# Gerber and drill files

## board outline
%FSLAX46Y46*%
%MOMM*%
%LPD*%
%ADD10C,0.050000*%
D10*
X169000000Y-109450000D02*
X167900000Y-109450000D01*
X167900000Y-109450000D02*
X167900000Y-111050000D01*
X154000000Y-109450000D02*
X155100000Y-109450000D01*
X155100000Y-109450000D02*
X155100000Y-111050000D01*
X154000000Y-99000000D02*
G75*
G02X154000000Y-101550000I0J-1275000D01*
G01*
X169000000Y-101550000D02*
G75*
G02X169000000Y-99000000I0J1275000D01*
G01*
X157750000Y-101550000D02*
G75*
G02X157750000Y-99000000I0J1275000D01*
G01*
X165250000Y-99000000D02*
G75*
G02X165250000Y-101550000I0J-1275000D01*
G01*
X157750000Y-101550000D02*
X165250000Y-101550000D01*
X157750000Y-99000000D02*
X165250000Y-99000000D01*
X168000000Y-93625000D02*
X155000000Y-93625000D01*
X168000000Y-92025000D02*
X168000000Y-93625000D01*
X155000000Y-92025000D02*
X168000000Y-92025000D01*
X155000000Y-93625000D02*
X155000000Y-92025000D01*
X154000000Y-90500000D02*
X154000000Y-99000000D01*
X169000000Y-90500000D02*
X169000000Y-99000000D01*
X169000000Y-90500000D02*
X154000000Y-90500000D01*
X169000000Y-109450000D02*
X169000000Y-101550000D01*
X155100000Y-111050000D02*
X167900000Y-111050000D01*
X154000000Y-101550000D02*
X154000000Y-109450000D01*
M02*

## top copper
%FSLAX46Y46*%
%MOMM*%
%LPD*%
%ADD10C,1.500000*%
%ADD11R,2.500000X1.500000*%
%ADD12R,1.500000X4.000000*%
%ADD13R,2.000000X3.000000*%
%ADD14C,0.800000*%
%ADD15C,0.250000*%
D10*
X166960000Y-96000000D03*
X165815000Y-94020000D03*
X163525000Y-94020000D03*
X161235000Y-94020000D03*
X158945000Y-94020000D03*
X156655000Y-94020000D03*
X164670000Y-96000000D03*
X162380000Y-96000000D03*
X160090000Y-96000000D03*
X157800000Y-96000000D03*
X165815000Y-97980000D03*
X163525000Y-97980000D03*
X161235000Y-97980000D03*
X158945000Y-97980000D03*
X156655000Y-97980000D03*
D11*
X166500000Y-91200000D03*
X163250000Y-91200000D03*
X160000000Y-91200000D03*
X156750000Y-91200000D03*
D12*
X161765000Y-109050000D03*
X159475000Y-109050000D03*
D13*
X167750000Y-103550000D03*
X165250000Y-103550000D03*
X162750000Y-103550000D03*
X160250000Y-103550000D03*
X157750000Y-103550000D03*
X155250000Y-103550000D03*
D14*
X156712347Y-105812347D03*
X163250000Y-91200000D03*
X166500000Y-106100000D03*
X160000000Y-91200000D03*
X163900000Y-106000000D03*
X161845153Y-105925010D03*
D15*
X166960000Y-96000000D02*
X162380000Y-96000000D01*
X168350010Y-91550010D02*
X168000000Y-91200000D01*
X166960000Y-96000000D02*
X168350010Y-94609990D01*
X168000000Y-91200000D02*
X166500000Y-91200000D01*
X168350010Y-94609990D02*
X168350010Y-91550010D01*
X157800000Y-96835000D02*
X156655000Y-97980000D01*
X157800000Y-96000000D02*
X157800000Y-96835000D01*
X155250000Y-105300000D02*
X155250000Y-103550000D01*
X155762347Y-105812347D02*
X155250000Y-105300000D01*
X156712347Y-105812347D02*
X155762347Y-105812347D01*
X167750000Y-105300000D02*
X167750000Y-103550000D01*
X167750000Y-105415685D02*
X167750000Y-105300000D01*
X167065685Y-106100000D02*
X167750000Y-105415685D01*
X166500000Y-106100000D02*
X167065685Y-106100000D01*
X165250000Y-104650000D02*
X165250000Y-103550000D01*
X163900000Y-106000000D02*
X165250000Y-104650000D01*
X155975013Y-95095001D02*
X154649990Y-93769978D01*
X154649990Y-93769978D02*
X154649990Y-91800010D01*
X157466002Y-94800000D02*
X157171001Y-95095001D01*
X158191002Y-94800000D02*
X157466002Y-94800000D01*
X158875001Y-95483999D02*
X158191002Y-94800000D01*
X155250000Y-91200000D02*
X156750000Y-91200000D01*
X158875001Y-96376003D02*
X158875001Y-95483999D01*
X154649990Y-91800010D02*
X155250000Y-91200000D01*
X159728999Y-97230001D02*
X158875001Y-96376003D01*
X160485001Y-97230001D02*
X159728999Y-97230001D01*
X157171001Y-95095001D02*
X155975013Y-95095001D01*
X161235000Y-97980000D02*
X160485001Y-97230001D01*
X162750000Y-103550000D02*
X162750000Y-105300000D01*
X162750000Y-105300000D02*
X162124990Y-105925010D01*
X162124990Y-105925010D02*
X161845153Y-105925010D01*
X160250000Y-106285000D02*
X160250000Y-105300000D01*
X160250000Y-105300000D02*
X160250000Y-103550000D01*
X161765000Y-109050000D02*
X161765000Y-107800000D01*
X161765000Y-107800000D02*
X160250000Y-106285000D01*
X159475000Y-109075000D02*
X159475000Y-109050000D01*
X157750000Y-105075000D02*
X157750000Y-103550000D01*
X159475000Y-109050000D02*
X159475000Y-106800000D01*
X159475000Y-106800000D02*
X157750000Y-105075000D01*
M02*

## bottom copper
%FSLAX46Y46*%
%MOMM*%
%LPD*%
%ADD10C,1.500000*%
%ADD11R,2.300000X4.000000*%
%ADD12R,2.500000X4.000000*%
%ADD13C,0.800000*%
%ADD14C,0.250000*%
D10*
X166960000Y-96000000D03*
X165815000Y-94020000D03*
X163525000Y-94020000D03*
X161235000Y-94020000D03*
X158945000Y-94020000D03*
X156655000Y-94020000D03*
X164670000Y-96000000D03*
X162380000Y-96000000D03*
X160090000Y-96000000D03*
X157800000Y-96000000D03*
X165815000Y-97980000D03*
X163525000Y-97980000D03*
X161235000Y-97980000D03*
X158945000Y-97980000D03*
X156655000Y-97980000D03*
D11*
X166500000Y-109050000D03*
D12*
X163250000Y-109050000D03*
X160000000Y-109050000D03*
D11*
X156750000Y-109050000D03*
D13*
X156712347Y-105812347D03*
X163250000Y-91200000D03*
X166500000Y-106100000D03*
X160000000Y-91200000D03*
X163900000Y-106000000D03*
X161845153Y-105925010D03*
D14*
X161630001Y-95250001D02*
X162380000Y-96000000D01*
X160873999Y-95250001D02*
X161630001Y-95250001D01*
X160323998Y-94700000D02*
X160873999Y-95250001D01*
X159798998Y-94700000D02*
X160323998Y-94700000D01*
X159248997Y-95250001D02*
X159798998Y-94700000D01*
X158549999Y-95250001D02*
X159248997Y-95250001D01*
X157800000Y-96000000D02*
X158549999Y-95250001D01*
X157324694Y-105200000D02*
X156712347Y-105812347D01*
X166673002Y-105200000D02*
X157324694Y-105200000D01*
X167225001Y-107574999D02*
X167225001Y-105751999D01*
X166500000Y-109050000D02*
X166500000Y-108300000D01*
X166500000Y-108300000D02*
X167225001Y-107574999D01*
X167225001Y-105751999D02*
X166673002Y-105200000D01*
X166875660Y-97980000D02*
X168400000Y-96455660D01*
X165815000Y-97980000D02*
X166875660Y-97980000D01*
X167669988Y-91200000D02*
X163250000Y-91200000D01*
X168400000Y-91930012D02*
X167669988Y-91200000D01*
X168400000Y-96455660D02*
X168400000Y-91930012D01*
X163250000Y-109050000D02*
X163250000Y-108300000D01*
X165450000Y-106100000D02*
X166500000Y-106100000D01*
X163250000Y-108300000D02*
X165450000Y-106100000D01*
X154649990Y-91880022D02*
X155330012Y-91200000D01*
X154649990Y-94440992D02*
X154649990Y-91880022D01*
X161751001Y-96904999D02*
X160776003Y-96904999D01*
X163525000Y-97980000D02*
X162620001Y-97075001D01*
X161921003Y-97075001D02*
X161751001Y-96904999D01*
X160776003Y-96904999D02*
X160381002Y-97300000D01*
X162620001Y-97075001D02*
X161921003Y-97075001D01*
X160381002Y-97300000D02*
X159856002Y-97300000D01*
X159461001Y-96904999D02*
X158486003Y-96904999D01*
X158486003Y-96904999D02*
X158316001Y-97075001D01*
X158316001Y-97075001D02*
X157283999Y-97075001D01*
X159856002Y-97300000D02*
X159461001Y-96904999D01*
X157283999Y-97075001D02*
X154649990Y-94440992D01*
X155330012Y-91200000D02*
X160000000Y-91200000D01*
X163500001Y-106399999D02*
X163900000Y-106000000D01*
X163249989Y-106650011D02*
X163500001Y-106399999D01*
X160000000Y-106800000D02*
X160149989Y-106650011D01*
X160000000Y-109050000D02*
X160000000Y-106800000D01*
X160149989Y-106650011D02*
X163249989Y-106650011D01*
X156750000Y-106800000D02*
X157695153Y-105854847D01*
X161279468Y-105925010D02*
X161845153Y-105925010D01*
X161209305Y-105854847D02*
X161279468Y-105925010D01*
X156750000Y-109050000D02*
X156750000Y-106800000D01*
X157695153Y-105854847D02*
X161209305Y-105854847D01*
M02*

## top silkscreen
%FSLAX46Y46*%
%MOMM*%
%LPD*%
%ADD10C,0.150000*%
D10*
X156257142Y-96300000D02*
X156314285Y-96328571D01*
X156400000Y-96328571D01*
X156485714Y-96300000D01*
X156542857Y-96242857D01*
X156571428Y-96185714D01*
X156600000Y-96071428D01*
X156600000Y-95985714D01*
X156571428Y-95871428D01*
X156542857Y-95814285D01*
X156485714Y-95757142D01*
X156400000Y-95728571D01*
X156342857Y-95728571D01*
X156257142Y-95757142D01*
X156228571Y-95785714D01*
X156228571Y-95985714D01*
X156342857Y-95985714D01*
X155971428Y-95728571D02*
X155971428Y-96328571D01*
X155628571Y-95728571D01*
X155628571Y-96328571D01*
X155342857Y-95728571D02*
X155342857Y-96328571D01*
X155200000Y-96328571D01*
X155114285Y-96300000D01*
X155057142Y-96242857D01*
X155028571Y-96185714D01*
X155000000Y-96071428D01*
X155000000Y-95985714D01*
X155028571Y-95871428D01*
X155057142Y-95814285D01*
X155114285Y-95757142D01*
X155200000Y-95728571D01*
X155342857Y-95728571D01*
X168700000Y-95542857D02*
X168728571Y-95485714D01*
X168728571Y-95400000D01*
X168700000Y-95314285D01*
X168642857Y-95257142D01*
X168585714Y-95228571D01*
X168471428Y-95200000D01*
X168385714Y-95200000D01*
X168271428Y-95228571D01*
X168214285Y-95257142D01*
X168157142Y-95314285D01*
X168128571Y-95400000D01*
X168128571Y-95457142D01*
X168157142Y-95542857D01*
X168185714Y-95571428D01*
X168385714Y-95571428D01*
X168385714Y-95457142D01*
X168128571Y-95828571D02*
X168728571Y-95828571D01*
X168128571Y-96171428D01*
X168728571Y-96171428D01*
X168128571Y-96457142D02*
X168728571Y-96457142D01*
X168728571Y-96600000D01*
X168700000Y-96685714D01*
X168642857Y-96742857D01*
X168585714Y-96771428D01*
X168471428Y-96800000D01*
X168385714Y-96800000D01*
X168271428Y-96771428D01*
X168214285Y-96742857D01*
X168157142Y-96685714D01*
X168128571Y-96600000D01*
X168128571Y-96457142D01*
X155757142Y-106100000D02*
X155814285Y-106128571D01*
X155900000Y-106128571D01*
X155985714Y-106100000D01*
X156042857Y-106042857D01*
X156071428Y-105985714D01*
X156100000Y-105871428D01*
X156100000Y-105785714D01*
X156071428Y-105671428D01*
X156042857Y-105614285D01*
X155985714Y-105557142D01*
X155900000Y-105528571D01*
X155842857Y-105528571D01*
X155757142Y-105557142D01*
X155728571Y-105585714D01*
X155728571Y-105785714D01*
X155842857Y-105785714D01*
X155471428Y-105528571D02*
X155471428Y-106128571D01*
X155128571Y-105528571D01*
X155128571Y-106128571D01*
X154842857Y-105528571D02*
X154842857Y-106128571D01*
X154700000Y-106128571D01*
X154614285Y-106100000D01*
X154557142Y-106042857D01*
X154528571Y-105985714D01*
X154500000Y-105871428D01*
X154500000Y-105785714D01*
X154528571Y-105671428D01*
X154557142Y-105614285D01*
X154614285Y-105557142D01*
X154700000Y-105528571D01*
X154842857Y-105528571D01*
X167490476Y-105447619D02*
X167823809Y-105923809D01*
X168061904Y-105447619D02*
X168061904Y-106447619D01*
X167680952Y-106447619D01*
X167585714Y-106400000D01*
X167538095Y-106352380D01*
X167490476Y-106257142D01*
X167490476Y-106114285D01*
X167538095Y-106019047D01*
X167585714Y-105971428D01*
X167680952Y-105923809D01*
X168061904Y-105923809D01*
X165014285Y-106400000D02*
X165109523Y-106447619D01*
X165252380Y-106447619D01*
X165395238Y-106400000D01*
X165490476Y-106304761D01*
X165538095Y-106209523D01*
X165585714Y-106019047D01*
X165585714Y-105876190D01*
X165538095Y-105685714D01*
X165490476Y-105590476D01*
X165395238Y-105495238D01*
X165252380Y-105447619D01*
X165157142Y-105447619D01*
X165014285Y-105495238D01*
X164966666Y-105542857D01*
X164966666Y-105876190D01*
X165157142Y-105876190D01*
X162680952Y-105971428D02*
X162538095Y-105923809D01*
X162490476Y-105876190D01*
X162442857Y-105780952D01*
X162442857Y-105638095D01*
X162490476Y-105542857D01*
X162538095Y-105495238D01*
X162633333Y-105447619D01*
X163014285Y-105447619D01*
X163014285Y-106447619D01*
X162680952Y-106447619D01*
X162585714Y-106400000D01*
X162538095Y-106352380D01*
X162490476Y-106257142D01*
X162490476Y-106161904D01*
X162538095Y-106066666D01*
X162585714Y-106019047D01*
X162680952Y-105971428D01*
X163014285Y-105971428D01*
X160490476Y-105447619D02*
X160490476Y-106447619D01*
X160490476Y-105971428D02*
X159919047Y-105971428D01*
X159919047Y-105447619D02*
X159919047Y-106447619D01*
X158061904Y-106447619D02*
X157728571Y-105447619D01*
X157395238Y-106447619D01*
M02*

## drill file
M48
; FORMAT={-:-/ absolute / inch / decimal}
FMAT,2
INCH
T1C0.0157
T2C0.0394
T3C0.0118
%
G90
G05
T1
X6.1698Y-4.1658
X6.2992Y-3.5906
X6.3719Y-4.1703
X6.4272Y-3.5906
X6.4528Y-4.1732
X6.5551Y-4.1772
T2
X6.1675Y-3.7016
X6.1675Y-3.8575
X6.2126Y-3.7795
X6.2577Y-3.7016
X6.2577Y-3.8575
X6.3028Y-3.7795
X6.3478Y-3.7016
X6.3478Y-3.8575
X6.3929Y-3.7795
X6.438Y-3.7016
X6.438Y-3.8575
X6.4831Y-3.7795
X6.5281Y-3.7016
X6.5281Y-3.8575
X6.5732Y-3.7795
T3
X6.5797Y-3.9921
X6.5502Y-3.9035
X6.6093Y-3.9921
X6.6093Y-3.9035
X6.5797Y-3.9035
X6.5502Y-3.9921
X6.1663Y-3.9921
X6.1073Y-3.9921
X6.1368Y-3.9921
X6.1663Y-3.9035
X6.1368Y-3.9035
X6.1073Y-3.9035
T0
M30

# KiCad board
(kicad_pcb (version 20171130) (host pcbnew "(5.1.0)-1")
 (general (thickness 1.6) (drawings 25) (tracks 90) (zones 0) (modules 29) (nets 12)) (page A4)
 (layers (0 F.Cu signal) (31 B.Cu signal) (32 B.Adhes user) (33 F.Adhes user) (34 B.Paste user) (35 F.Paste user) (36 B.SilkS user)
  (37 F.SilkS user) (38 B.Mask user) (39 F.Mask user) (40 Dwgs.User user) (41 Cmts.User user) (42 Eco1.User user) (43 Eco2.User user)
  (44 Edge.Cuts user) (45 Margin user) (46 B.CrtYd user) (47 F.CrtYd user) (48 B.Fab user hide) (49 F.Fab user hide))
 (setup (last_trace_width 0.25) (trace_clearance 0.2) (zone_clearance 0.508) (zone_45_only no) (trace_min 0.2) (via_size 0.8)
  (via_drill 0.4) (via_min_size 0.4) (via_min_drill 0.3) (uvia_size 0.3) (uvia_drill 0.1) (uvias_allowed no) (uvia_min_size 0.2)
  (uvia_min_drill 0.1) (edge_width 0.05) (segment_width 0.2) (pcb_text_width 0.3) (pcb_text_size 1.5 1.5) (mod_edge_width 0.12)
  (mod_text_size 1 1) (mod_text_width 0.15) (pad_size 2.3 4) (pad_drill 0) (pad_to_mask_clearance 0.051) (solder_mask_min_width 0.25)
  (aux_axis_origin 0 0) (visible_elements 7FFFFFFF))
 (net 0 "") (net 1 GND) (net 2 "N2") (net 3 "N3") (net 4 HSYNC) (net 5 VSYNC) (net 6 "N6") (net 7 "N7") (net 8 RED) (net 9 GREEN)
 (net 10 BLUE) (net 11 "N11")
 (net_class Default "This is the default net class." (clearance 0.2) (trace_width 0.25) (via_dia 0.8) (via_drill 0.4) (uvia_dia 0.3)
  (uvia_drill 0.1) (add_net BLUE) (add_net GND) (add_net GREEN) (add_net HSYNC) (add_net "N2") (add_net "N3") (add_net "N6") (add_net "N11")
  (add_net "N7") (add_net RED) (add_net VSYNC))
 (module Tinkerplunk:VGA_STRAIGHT (layer B.Cu) (at 161.5 96 180)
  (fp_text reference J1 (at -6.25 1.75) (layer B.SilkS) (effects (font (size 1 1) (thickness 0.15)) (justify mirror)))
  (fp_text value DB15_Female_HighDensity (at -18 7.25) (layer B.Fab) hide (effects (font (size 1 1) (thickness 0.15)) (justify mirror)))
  (pad 6 thru_hole circle (at -5.46 0 180) (size 1.5 1.5) (drill 1) (layers *.Cu *.Mask) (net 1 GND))
  (pad 11 thru_hole circle (at -4.315 1.98 180) (size 1.5 1.5) (drill 1) (layers *.Cu *.Mask) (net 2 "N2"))
  (pad 12 thru_hole circle (at -2.025 1.98 180) (size 1.5 1.5) (drill 1) (layers *.Cu *.Mask) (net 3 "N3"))
  (pad 13 thru_hole circle (at 0.265 1.98 180) (size 1.5 1.5) (drill 1) (layers *.Cu *.Mask) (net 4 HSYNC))
  (pad 14 thru_hole circle (at 2.555 1.98 180) (size 1.5 1.5) (drill 1) (layers *.Cu *.Mask) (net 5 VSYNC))
  (pad 15 thru_hole circle (at 4.845 1.98 180) (size 1.5 1.5) (drill 1) (layers *.Cu *.Mask) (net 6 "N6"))
  (pad 7 thru_hole circle (at -3.17 0 180) (size 1.5 1.5) (drill 1) (layers *.Cu *.Mask) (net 1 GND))
  (pad 8 thru_hole circle (at -0.88 0 180) (size 1.5 1.5) (drill 1) (layers *.Cu *.Mask) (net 1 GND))
  (pad 9 thru_hole circle (at 1.41 0 180) (size 1.5 1.5) (drill 1) (layers *.Cu *.Mask) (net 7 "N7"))
  (pad 10 thru_hole circle (at 3.7 0 180) (size 1.5 1.5) (drill 1) (layers *.Cu *.Mask) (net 1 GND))
  (pad 1 thru_hole circle (at -4.315 -1.98 180) (size 1.5 1.5) (drill 1) (layers *.Cu *.Mask) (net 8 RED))
  (pad 2 thru_hole circle (at -2.025 -1.98 180) (size 1.5 1.5) (drill 1) (layers *.Cu *.Mask) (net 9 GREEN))
  (pad 3 thru_hole circle (at 0.265 -1.98 180) (size 1.5 1.5) (drill 1) (layers *.Cu *.Mask) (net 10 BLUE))
  (pad 4 thru_hole circle (at 2.555 -1.98 180) (size 1.5 1.5) (drill 1) (layers *.Cu *.Mask) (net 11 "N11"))
  (pad 5 thru_hole circle (at 4.845 -1.98 180) (size 1.5 1.5) (drill 1) (layers *.Cu *.Mask) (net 1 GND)))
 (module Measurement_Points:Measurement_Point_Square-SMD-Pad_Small (layer B.Cu) (at 166.5 109.05)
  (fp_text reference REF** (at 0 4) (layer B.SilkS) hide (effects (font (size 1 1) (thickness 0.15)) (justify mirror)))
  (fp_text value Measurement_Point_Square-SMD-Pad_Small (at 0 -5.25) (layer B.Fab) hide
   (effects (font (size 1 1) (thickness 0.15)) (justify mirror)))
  (pad 1 smd rect (at 0 0) (size 2.3 4) (layers B.Cu B.Mask) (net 1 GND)))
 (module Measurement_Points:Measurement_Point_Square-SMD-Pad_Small (layer B.Cu) (at 163.25 109.05)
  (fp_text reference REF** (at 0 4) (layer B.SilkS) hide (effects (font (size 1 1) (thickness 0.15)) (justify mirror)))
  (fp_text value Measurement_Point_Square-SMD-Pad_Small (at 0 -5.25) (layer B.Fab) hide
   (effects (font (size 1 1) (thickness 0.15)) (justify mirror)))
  (pad 1 smd rect (at 0 0) (size 2.5 4) (layers B.Cu B.Mask) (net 8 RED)))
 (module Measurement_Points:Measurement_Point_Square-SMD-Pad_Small (layer B.Cu) (at 160 109.05)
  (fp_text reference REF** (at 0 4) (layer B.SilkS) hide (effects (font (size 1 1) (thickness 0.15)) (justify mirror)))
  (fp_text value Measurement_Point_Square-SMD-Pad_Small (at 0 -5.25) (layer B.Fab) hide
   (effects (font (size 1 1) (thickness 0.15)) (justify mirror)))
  (pad 1 smd rect (at 0 0) (size 2.5 4) (layers B.Cu B.Mask) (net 9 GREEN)))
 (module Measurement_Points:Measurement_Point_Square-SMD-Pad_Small (layer B.Cu) (at 156.75 109.05)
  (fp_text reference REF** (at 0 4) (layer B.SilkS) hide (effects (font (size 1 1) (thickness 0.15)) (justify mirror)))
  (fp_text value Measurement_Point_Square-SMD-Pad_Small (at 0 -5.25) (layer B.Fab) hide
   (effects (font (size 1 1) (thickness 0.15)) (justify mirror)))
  (pad 1 smd rect (at 0 0) (size 2.3 4) (layers B.Cu B.Mask) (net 10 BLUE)))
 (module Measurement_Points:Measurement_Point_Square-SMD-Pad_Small (layer F.Cu) (at 166.5 91.2 90)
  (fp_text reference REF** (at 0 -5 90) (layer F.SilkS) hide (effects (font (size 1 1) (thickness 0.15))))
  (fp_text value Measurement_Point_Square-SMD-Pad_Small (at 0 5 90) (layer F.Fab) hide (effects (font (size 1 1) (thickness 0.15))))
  (pad 1 smd rect (at 0 0 90) (size 1.5 2.5) (layers F.Cu F.Mask) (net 1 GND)))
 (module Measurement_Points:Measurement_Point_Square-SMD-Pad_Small (layer F.Cu) (at 163.25 91.2 90)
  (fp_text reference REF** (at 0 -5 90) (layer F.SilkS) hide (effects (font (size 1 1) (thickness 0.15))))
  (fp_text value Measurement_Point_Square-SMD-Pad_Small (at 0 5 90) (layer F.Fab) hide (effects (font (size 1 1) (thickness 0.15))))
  (pad 1 smd rect (at 0 0 90) (size 1.5 2.5) (layers F.Cu F.Mask) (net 8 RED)))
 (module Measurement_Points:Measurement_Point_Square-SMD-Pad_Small (layer F.Cu) (at 160 91.2 90)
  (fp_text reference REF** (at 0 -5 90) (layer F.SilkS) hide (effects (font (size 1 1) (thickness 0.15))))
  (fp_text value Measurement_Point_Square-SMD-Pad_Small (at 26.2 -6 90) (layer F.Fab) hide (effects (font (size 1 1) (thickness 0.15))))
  (pad 1 smd rect (at 0 0 90) (size 1.5 2.5) (layers F.Cu F.Mask) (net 9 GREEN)))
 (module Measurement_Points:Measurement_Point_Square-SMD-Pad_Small (layer F.Cu) (at 156.75 91.2 90)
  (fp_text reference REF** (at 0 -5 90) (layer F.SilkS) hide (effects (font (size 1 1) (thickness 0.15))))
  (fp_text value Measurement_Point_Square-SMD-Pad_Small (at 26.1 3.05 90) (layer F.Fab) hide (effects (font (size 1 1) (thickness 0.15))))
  (pad 1 smd rect (at 0 0 90) (size 1.5 2.5) (layers F.Cu F.Mask) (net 10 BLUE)))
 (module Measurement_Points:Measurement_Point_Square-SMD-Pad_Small (layer F.Cu) (at 161.765 109.05)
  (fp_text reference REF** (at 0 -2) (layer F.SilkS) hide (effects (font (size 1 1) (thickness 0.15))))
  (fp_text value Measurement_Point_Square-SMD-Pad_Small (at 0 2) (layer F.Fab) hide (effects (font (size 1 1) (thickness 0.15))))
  (pad 1 smd rect (at 0 0) (size 1.5 4) (layers F.Cu F.Mask) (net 4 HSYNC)))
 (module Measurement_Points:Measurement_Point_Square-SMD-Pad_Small (layer F.Cu) (at 159.475 109.05)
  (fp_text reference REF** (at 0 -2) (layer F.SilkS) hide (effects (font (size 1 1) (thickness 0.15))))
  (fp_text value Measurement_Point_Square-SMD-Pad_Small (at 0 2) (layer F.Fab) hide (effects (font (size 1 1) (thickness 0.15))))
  (pad 1 smd rect (at 0 0) (size 1.5 4) (layers F.Cu F.Mask) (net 5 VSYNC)))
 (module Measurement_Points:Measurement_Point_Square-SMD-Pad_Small (layer F.Cu) (at 167.75 103.55)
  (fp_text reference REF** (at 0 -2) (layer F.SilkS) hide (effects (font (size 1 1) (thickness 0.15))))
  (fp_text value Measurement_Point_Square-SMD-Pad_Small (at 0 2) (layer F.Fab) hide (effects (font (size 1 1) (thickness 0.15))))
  (pad 1 smd rect (at 0 0) (size 2 3) (layers F.Cu F.Mask) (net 8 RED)))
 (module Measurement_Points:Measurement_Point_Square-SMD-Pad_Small (layer F.Cu) (at 165.25 103.55)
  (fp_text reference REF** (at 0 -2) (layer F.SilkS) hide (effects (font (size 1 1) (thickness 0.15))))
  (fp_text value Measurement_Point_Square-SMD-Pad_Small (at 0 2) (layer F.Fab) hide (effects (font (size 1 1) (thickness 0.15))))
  (pad 1 smd rect (at 0 0) (size 2 3) (layers F.Cu F.Mask) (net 9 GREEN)))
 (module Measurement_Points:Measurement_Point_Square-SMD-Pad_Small (layer F.Cu) (at 162.75 103.55)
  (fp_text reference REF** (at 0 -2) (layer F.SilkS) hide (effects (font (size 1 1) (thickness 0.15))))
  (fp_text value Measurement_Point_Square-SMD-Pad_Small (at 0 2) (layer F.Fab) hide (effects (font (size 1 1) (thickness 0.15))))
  (pad 1 smd rect (at 0 0) (size 2 3) (layers F.Cu F.Mask) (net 10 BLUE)))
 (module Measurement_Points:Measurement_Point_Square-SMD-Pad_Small (layer F.Cu) (at 160.25 103.55)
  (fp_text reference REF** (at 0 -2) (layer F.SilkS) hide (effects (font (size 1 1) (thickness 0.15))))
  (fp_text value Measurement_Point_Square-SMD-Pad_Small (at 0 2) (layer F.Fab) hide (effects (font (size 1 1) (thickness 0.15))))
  (pad 1 smd rect (at 0 0) (size 2 3) (layers F.Cu F.Mask) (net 4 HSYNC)))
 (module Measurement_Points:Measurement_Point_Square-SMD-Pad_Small (layer F.Cu) (at 157.75 103.55)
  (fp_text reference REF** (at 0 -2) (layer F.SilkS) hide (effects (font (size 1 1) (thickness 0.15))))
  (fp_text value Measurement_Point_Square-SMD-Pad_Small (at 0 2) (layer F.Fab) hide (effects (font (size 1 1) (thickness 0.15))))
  (pad 1 smd rect (at 0 0) (size 2 3) (layers F.Cu F.Mask) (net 5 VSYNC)))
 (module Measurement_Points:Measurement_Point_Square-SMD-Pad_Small (layer F.Cu) (at 155.25 103.55)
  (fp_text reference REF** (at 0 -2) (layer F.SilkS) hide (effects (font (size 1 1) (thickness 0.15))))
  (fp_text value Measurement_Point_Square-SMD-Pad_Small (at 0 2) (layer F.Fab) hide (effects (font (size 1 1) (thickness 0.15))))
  (pad 1 smd rect (at 0 0) (size 2 3) (layers F.Cu F.Mask) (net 1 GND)))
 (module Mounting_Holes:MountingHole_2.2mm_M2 (layer F.Cu) (at 167.125 99.75)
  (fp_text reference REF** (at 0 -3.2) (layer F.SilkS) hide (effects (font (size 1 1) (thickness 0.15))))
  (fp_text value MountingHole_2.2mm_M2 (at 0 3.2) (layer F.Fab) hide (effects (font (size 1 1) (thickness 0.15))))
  (pad "" np_thru_hole circle (at 0 1.65) (size 0.3 0.3) (drill 0.3) (layers *.Cu *.Mask)))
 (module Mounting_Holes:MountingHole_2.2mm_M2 (layer F.Cu) (at 166.375 99.15)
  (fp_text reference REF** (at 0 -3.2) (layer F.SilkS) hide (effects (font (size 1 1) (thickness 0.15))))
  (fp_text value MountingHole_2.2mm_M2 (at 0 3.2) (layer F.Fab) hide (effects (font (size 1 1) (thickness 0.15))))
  (pad "" np_thru_hole circle (at 0 0) (size 0.3 0.3) (drill 0.3) (layers *.Cu *.Mask)))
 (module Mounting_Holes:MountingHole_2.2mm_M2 (layer F.Cu) (at 167.875 99.75)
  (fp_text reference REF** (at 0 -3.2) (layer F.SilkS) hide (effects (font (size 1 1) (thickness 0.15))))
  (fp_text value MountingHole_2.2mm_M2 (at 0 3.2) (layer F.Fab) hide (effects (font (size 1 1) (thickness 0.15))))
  (pad "" np_thru_hole circle (at 0 1.65) (size 0.3 0.3) (drill 0.3) (layers *.Cu *.Mask)))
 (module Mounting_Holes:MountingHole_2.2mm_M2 (layer F.Cu) (at 168.25 99.15)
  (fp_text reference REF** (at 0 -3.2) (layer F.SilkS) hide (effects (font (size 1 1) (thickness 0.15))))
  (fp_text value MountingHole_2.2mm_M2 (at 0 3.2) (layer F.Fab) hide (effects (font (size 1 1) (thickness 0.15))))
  (pad "" np_thru_hole circle (at -0.375 0) (size 0.3 0.3) (drill 0.3) (layers *.Cu *.Mask)))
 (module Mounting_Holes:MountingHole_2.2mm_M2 (layer F.Cu) (at 167.125 99.15)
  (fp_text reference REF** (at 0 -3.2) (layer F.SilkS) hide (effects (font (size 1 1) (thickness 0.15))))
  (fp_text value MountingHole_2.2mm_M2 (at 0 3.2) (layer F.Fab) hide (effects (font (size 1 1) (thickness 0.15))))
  (pad "" np_thru_hole circle (at 0 0) (size 0.3 0.3) (drill 0.3) (layers *.Cu *.Mask)))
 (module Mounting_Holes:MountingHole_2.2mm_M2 (layer F.Cu) (at 166.375 101.4)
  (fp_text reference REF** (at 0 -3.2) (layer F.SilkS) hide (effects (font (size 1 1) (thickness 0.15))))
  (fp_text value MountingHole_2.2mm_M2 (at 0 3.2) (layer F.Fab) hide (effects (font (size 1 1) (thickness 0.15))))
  (pad "" np_thru_hole circle (at 0 0) (size 0.3 0.3) (drill 0.3) (layers *.Cu *.Mask)))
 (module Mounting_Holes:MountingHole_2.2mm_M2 (layer F.Cu) (at 155.125 101.45)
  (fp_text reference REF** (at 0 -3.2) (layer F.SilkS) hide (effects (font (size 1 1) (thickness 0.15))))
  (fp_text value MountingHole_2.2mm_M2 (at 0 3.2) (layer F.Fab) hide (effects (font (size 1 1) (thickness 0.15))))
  (pad "" np_thru_hole circle (at 0 -0.05) (size 0.3 0.3) (drill 0.3) (layers *.Cu *.Mask)))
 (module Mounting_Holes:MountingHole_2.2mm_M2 (layer F.Cu) (at 156.625 101.45)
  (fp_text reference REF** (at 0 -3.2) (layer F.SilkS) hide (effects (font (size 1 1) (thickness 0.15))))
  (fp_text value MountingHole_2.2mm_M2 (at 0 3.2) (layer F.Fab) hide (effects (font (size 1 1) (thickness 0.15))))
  (pad "" np_thru_hole circle (at 0 -0.05) (size 0.3 0.3) (drill 0.3) (layers *.Cu *.Mask)))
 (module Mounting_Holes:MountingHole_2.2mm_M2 (layer F.Cu) (at 155.875 101.45)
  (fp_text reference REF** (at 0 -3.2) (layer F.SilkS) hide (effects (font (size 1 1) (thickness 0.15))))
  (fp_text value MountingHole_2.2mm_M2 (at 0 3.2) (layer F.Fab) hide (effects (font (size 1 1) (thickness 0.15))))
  (pad "" np_thru_hole circle (at 0 -0.05) (size 0.3 0.3) (drill 0.3) (layers *.Cu *.Mask)))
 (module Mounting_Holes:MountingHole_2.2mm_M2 (layer F.Cu) (at 156.625 99.15)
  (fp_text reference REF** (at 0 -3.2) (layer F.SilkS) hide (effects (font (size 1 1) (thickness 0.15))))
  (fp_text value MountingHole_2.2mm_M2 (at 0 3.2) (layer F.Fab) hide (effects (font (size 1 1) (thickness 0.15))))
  (pad "" np_thru_hole circle (at 0 0) (size 0.3 0.3) (drill 0.3) (layers *.Cu *.Mask)))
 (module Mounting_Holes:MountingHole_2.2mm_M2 (layer F.Cu) (at 155.875 99.15)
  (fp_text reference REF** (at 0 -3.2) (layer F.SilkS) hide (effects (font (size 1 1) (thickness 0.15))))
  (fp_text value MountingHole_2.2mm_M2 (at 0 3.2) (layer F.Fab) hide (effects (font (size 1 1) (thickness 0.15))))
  (pad "" np_thru_hole circle (at 0 0) (size 0.3 0.3) (drill 0.3) (layers *.Cu *.Mask)))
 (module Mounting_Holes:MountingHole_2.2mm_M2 (layer F.Cu) (at 155.125 99.15)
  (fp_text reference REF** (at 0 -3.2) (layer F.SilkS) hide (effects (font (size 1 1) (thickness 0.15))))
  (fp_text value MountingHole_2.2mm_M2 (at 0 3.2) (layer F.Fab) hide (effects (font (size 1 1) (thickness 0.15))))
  (pad "" np_thru_hole circle (at 0 0) (size 0.3 0.3) (drill 0.3) (layers *.Cu *.Mask)))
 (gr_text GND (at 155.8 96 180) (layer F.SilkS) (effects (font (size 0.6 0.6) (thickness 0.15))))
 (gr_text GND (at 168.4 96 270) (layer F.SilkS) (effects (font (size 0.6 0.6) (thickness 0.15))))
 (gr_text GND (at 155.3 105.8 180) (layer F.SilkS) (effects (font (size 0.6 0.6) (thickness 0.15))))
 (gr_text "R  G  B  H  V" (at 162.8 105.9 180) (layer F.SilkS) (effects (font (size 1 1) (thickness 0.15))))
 (gr_line (start 169 109.45) (end 167.9 109.45) (layer Edge.Cuts) (width 0.05))
 (gr_line (start 167.9 109.45) (end 167.9 111.05) (layer Edge.Cuts) (width 0.05))
 (gr_line (start 154 109.45) (end 155.1 109.45) (layer Edge.Cuts) (width 0.05))
 (gr_line (start 155.1 109.45) (end 155.1 111.05) (layer Edge.Cuts) (width 0.05))
 (gr_arc (start 154 100.275) (end 154 101.55) (angle -180) (layer Edge.Cuts) (width 0.05))
 (gr_arc (start 169 100.275) (end 169 99) (angle -180) (layer Edge.Cuts) (width 0.05))
 (gr_arc (start 157.75 100.275) (end 157.75 99) (angle -180) (layer Edge.Cuts) (width 0.05))
 (gr_arc (start 165.25 100.275) (end 165.25 101.55) (angle -180) (layer Edge.Cuts) (width 0.05))
 (gr_line (start 157.75 101.55) (end 165.25 101.55) (layer Edge.Cuts) (width 0.05))
 (gr_line (start 157.75 99) (end 165.25 99) (layer Edge.Cuts) (width 0.05))
 (gr_line (start 168 93.625) (end 155 93.625) (layer Edge.Cuts) (width 0.05))
 (gr_line (start 168 92.025) (end 168 93.625) (layer Edge.Cuts) (width 0.05))
 (gr_line (start 155 92.025) (end 168 92.025) (layer Edge.Cuts) (width 0.05))
 (gr_line (start 155 93.625) (end 155 92.025) (layer Edge.Cuts) (width 0.05))
 (gr_line (start 154 90.5) (end 154 99) (layer Edge.Cuts) (width 0.05))
 (gr_line (start 169 90.5) (end 169 99) (layer Edge.Cuts) (width 0.05))
 (gr_line (start 169 90.5) (end 154 90.5) (layer Edge.Cuts) (width 0.05))
 (gr_line (start 169 109.45) (end 169 101.55) (layer Edge.Cuts) (width 0.05))
 (gr_line (start 155.1 111.05) (end 167.9 111.05) (layer Edge.Cuts) (width 0.05))
 (gr_line (start 154 101.55) (end 154 109.45) (layer Edge.Cuts) (width 0.05))
 (segment (start 166.96 96) (end 162.38 96) (width 0.25) (layer F.Cu) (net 1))
 (segment (start 168.35001 91.55001) (end 168 91.2) (width 0.25) (layer F.Cu) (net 1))
 (segment (start 166.96 96) (end 168.35001 94.60999) (width 0.25) (layer F.Cu) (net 1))
 (segment (start 168 91.2) (end 166.5 91.2) (width 0.25) (layer F.Cu) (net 1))
 (segment (start 168.35001 94.60999) (end 168.35001 91.55001) (width 0.25) (layer F.Cu) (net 1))
 (segment (start 157.8 96.835) (end 156.655 97.98) (width 0.25) (layer F.Cu) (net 1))
 (segment (start 157.8 96) (end 157.8 96.835) (width 0.25) (layer F.Cu) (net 1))
 (segment (start 161.630001 95.250001) (end 162.38 96) (width 0.25) (layer B.Cu) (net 1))
 (segment (start 160.873999 95.250001) (end 161.630001 95.250001) (width 0.25) (layer B.Cu) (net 1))
 (segment (start 160.323998 94.7) (end 160.873999 95.250001) (width 0.25) (layer B.Cu) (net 1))
 (segment (start 159.798998 94.7) (end 160.323998 94.7) (width 0.25) (layer B.Cu) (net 1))
 (segment (start 159.248997 95.250001) (end 159.798998 94.7) (width 0.25) (layer B.Cu) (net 1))
 (segment (start 158.549999 95.250001) (end 159.248997 95.250001) (width 0.25) (layer B.Cu) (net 1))
 (segment (start 157.8 96) (end 158.549999 95.250001) (width 0.25) (layer B.Cu) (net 1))
 (via (at 156.712347 105.812347) (size 0.8) (drill 0.4) (layers F.Cu B.Cu) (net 1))
 (segment (start 155.25 105.3) (end 155.25 103.55) (width 0.25) (layer F.Cu) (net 1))
 (segment (start 155.762347 105.812347) (end 155.25 105.3) (width 0.25) (layer F.Cu) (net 1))
 (segment (start 156.712347 105.812347) (end 155.762347 105.812347) (width 0.25) (layer F.Cu) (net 1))
 (segment (start 157.324694 105.2) (end 156.712347 105.812347) (width 0.25) (layer B.Cu) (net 1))
 (segment (start 166.673002 105.2) (end 157.324694 105.2) (width 0.25) (layer B.Cu) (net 1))
 (segment (start 167.225001 107.574999) (end 167.225001 105.751999) (width 0.25) (layer B.Cu) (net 1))
 (segment (start 166.5 109.05) (end 166.5 108.3) (width 0.25) (layer B.Cu) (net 1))
 (segment (start 166.5 108.3) (end 167.225001 107.574999) (width 0.25) (layer B.Cu) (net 1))
 (segment (start 167.225001 105.751999) (end 166.673002 105.2) (width 0.25) (layer B.Cu) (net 1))
 (segment (start 166.87566 97.98) (end 168.4 96.45566) (width 0.25) (layer B.Cu) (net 8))
 (segment (start 165.815 97.98) (end 166.87566 97.98) (width 0.25) (layer B.Cu) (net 8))
 (via (at 163.25 91.2) (size 0.8) (drill 0.4) (layers F.Cu B.Cu) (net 8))
 (segment (start 167.669988 91.2) (end 163.25 91.2) (width 0.25) (layer B.Cu) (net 8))
 (segment (start 168.4 91.930012) (end 167.669988 91.2) (width 0.25) (layer B.Cu) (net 8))
 (segment (start 168.4 96.45566) (end 168.4 91.930012) (width 0.25) (layer B.Cu) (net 8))
 (segment (start 163.25 109.05) (end 163.25 108.3) (width 0.25) (layer B.Cu) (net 8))
 (via (at 166.5 106.1) (size 0.8) (drill 0.4) (layers F.Cu B.Cu) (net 8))
 (segment (start 165.45 106.1) (end 166.5 106.1) (width 0.25) (layer B.Cu) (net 8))
 (segment (start 163.25 108.3) (end 165.45 106.1) (width 0.25) (layer B.Cu) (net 8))
 (segment (start 167.75 105.3) (end 167.75 103.55) (width 0.25) (layer F.Cu) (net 8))
 (segment (start 167.75 105.415685) (end 167.75 105.3) (width 0.25) (layer F.Cu) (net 8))
 (segment (start 167.065685 106.1) (end 167.75 105.415685) (width 0.25) (layer F.Cu) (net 8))
 (segment (start 166.5 106.1) (end 167.065685 106.1) (width 0.25) (layer F.Cu) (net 8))
 (segment (start 154.64999 91.880022) (end 155.330012 91.2) (width 0.25) (layer B.Cu) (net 9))
 (segment (start 154.64999 94.440992) (end 154.64999 91.880022) (width 0.25) (layer B.Cu) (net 9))
 (segment (start 161.751001 96.904999) (end 160.776003 96.904999) (width 0.25) (layer B.Cu) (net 9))
 (segment (start 163.525 97.98) (end 162.620001 97.075001) (width 0.25) (layer B.Cu) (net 9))
 (segment (start 161.921003 97.075001) (end 161.751001 96.904999) (width 0.25) (layer B.Cu) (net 9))
 (segment (start 160.776003 96.904999) (end 160.381002 97.3) (width 0.25) (layer B.Cu) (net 9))
 (segment (start 162.620001 97.075001) (end 161.921003 97.075001) (width 0.25) (layer B.Cu) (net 9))
 (segment (start 160.381002 97.3) (end 159.856002 97.3) (width 0.25) (layer B.Cu) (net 9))
 (segment (start 159.461001 96.904999) (end 158.486003 96.904999) (width 0.25) (layer B.Cu) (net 9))
 (segment (start 158.486003 96.904999) (end 158.316001 97.075001) (width 0.25) (layer B.Cu) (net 9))
 (segment (start 158.316001 97.075001) (end 157.283999 97.075001) (width 0.25) (layer B.Cu) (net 9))
 (segment (start 159.856002 97.3) (end 159.461001 96.904999) (width 0.25) (layer B.Cu) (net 9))
 (segment (start 157.283999 97.075001) (end 154.64999 94.440992) (width 0.25) (layer B.Cu) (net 9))
 (segment (start 155.330012 91.2) (end 160 91.2) (width 0.25) (layer B.Cu) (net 9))
 (via (at 160 91.2) (size 0.8) (drill 0.4) (layers F.Cu B.Cu) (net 9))
 (via (at 163.9 106) (size 0.8) (drill 0.4) (layers F.Cu B.Cu) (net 9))
 (segment (start 165.25 104.65) (end 165.25 103.55) (width 0.25) (layer F.Cu) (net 9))
 (segment (start 163.9 106) (end 165.25 104.65) (width 0.25) (layer F.Cu) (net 9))
 (segment (start 163.500001 106.399999) (end 163.9 106) (width 0.25) (layer B.Cu) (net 9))
 (segment (start 163.249989 106.650011) (end 163.500001 106.399999) (width 0.25) (layer B.Cu) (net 9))
 (segment (start 160 106.8) (end 160.149989 106.650011) (width 0.25) (layer B.Cu) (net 9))
 (segment (start 160 109.05) (end 160 106.8) (width 0.25) (layer B.Cu) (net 9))
 (segment (start 160.149989 106.650011) (end 163.249989 106.650011) (width 0.25) (layer B.Cu) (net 9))
 (segment (start 155.975013 95.095001) (end 154.64999 93.769978) (width 0.25) (layer F.Cu) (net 10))
 (segment (start 154.64999 93.769978) (end 154.64999 91.80001) (width 0.25) (layer F.Cu) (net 10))
 (segment (start 157.466002 94.8) (end 157.171001 95.095001) (width 0.25) (layer F.Cu) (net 10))
 (segment (start 158.191002 94.8) (end 157.466002 94.8) (width 0.25) (layer F.Cu) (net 10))
 (segment (start 158.875001 95.483999) (end 158.191002 94.8) (width 0.25) (layer F.Cu) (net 10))
 (segment (start 155.25 91.2) (end 156.75 91.2) (width 0.25) (layer F.Cu) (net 10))
 (segment (start 158.875001 96.376003) (end 158.875001 95.483999) (width 0.25) (layer F.Cu) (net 10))
 (segment (start 154.64999 91.80001) (end 155.25 91.2) (width 0.25) (layer F.Cu) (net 10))
 (segment (start 159.728999 97.230001) (end 158.875001 96.376003) (width 0.25) (layer F.Cu) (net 10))
 (segment (start 160.485001 97.230001) (end 159.728999 97.230001) (width 0.25) (layer F.Cu) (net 10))
 (segment (start 157.171001 95.095001) (end 155.975013 95.095001) (width 0.25) (layer F.Cu) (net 10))
 (segment (start 161.235 97.98) (end 160.485001 97.230001) (width 0.25) (layer F.Cu) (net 10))
 (segment (start 162.75 103.55) (end 162.75 105.3) (width 0.25) (layer F.Cu) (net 10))
 (segment (start 156.75 106.8) (end 157.695153 105.854847) (width 0.25) (layer B.Cu) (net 10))
 (segment (start 162.75 105.3) (end 162.12499 105.92501) (width 0.25) (layer F.Cu) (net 10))
 (segment (start 161.279468 105.92501) (end 161.845153 105.92501) (width 0.25) (layer B.Cu) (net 10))
 (segment (start 161.209305 105.854847) (end 161.279468 105.92501) (width 0.25) (layer B.Cu) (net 10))
 (segment (start 156.75 109.05) (end 156.75 106.8) (width 0.25) (layer B.Cu) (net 10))
 (segment (start 157.695153 105.854847) (end 161.209305 105.854847) (width 0.25) (layer B.Cu) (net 10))
 (via (at 161.845153 105.92501) (size 0.8) (drill 0.4) (layers F.Cu B.Cu) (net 10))
 (segment (start 162.12499 105.92501) (end 161.845153 105.92501) (width 0.25) (layer F.Cu) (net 10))
 (segment (start 160.25 106.285) (end 160.25 105.3) (width 0.25) (layer F.Cu) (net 4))
 (segment (start 160.25 105.3) (end 160.25 103.55) (width 0.25) (layer F.Cu) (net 4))
 (segment (start 161.765 109.05) (end 161.765 107.8) (width 0.25) (layer F.Cu) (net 4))
 (segment (start 161.765 107.8) (end 160.25 106.285) (width 0.25) (layer F.Cu) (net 4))
 (segment (start 159.475 109.075) (end 159.475 109.05) (width 0.25) (layer F.Cu) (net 5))
 (segment (start 157.75 105.075) (end 157.75 103.55) (width 0.25) (layer F.Cu) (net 5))
 (segment (start 159.475 109.05) (end 159.475 106.8) (width 0.25) (layer F.Cu) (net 5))
 (segment (start 159.475 106.8) (end 157.75 105.075) (width 0.25) (layer F.Cu) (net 5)))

